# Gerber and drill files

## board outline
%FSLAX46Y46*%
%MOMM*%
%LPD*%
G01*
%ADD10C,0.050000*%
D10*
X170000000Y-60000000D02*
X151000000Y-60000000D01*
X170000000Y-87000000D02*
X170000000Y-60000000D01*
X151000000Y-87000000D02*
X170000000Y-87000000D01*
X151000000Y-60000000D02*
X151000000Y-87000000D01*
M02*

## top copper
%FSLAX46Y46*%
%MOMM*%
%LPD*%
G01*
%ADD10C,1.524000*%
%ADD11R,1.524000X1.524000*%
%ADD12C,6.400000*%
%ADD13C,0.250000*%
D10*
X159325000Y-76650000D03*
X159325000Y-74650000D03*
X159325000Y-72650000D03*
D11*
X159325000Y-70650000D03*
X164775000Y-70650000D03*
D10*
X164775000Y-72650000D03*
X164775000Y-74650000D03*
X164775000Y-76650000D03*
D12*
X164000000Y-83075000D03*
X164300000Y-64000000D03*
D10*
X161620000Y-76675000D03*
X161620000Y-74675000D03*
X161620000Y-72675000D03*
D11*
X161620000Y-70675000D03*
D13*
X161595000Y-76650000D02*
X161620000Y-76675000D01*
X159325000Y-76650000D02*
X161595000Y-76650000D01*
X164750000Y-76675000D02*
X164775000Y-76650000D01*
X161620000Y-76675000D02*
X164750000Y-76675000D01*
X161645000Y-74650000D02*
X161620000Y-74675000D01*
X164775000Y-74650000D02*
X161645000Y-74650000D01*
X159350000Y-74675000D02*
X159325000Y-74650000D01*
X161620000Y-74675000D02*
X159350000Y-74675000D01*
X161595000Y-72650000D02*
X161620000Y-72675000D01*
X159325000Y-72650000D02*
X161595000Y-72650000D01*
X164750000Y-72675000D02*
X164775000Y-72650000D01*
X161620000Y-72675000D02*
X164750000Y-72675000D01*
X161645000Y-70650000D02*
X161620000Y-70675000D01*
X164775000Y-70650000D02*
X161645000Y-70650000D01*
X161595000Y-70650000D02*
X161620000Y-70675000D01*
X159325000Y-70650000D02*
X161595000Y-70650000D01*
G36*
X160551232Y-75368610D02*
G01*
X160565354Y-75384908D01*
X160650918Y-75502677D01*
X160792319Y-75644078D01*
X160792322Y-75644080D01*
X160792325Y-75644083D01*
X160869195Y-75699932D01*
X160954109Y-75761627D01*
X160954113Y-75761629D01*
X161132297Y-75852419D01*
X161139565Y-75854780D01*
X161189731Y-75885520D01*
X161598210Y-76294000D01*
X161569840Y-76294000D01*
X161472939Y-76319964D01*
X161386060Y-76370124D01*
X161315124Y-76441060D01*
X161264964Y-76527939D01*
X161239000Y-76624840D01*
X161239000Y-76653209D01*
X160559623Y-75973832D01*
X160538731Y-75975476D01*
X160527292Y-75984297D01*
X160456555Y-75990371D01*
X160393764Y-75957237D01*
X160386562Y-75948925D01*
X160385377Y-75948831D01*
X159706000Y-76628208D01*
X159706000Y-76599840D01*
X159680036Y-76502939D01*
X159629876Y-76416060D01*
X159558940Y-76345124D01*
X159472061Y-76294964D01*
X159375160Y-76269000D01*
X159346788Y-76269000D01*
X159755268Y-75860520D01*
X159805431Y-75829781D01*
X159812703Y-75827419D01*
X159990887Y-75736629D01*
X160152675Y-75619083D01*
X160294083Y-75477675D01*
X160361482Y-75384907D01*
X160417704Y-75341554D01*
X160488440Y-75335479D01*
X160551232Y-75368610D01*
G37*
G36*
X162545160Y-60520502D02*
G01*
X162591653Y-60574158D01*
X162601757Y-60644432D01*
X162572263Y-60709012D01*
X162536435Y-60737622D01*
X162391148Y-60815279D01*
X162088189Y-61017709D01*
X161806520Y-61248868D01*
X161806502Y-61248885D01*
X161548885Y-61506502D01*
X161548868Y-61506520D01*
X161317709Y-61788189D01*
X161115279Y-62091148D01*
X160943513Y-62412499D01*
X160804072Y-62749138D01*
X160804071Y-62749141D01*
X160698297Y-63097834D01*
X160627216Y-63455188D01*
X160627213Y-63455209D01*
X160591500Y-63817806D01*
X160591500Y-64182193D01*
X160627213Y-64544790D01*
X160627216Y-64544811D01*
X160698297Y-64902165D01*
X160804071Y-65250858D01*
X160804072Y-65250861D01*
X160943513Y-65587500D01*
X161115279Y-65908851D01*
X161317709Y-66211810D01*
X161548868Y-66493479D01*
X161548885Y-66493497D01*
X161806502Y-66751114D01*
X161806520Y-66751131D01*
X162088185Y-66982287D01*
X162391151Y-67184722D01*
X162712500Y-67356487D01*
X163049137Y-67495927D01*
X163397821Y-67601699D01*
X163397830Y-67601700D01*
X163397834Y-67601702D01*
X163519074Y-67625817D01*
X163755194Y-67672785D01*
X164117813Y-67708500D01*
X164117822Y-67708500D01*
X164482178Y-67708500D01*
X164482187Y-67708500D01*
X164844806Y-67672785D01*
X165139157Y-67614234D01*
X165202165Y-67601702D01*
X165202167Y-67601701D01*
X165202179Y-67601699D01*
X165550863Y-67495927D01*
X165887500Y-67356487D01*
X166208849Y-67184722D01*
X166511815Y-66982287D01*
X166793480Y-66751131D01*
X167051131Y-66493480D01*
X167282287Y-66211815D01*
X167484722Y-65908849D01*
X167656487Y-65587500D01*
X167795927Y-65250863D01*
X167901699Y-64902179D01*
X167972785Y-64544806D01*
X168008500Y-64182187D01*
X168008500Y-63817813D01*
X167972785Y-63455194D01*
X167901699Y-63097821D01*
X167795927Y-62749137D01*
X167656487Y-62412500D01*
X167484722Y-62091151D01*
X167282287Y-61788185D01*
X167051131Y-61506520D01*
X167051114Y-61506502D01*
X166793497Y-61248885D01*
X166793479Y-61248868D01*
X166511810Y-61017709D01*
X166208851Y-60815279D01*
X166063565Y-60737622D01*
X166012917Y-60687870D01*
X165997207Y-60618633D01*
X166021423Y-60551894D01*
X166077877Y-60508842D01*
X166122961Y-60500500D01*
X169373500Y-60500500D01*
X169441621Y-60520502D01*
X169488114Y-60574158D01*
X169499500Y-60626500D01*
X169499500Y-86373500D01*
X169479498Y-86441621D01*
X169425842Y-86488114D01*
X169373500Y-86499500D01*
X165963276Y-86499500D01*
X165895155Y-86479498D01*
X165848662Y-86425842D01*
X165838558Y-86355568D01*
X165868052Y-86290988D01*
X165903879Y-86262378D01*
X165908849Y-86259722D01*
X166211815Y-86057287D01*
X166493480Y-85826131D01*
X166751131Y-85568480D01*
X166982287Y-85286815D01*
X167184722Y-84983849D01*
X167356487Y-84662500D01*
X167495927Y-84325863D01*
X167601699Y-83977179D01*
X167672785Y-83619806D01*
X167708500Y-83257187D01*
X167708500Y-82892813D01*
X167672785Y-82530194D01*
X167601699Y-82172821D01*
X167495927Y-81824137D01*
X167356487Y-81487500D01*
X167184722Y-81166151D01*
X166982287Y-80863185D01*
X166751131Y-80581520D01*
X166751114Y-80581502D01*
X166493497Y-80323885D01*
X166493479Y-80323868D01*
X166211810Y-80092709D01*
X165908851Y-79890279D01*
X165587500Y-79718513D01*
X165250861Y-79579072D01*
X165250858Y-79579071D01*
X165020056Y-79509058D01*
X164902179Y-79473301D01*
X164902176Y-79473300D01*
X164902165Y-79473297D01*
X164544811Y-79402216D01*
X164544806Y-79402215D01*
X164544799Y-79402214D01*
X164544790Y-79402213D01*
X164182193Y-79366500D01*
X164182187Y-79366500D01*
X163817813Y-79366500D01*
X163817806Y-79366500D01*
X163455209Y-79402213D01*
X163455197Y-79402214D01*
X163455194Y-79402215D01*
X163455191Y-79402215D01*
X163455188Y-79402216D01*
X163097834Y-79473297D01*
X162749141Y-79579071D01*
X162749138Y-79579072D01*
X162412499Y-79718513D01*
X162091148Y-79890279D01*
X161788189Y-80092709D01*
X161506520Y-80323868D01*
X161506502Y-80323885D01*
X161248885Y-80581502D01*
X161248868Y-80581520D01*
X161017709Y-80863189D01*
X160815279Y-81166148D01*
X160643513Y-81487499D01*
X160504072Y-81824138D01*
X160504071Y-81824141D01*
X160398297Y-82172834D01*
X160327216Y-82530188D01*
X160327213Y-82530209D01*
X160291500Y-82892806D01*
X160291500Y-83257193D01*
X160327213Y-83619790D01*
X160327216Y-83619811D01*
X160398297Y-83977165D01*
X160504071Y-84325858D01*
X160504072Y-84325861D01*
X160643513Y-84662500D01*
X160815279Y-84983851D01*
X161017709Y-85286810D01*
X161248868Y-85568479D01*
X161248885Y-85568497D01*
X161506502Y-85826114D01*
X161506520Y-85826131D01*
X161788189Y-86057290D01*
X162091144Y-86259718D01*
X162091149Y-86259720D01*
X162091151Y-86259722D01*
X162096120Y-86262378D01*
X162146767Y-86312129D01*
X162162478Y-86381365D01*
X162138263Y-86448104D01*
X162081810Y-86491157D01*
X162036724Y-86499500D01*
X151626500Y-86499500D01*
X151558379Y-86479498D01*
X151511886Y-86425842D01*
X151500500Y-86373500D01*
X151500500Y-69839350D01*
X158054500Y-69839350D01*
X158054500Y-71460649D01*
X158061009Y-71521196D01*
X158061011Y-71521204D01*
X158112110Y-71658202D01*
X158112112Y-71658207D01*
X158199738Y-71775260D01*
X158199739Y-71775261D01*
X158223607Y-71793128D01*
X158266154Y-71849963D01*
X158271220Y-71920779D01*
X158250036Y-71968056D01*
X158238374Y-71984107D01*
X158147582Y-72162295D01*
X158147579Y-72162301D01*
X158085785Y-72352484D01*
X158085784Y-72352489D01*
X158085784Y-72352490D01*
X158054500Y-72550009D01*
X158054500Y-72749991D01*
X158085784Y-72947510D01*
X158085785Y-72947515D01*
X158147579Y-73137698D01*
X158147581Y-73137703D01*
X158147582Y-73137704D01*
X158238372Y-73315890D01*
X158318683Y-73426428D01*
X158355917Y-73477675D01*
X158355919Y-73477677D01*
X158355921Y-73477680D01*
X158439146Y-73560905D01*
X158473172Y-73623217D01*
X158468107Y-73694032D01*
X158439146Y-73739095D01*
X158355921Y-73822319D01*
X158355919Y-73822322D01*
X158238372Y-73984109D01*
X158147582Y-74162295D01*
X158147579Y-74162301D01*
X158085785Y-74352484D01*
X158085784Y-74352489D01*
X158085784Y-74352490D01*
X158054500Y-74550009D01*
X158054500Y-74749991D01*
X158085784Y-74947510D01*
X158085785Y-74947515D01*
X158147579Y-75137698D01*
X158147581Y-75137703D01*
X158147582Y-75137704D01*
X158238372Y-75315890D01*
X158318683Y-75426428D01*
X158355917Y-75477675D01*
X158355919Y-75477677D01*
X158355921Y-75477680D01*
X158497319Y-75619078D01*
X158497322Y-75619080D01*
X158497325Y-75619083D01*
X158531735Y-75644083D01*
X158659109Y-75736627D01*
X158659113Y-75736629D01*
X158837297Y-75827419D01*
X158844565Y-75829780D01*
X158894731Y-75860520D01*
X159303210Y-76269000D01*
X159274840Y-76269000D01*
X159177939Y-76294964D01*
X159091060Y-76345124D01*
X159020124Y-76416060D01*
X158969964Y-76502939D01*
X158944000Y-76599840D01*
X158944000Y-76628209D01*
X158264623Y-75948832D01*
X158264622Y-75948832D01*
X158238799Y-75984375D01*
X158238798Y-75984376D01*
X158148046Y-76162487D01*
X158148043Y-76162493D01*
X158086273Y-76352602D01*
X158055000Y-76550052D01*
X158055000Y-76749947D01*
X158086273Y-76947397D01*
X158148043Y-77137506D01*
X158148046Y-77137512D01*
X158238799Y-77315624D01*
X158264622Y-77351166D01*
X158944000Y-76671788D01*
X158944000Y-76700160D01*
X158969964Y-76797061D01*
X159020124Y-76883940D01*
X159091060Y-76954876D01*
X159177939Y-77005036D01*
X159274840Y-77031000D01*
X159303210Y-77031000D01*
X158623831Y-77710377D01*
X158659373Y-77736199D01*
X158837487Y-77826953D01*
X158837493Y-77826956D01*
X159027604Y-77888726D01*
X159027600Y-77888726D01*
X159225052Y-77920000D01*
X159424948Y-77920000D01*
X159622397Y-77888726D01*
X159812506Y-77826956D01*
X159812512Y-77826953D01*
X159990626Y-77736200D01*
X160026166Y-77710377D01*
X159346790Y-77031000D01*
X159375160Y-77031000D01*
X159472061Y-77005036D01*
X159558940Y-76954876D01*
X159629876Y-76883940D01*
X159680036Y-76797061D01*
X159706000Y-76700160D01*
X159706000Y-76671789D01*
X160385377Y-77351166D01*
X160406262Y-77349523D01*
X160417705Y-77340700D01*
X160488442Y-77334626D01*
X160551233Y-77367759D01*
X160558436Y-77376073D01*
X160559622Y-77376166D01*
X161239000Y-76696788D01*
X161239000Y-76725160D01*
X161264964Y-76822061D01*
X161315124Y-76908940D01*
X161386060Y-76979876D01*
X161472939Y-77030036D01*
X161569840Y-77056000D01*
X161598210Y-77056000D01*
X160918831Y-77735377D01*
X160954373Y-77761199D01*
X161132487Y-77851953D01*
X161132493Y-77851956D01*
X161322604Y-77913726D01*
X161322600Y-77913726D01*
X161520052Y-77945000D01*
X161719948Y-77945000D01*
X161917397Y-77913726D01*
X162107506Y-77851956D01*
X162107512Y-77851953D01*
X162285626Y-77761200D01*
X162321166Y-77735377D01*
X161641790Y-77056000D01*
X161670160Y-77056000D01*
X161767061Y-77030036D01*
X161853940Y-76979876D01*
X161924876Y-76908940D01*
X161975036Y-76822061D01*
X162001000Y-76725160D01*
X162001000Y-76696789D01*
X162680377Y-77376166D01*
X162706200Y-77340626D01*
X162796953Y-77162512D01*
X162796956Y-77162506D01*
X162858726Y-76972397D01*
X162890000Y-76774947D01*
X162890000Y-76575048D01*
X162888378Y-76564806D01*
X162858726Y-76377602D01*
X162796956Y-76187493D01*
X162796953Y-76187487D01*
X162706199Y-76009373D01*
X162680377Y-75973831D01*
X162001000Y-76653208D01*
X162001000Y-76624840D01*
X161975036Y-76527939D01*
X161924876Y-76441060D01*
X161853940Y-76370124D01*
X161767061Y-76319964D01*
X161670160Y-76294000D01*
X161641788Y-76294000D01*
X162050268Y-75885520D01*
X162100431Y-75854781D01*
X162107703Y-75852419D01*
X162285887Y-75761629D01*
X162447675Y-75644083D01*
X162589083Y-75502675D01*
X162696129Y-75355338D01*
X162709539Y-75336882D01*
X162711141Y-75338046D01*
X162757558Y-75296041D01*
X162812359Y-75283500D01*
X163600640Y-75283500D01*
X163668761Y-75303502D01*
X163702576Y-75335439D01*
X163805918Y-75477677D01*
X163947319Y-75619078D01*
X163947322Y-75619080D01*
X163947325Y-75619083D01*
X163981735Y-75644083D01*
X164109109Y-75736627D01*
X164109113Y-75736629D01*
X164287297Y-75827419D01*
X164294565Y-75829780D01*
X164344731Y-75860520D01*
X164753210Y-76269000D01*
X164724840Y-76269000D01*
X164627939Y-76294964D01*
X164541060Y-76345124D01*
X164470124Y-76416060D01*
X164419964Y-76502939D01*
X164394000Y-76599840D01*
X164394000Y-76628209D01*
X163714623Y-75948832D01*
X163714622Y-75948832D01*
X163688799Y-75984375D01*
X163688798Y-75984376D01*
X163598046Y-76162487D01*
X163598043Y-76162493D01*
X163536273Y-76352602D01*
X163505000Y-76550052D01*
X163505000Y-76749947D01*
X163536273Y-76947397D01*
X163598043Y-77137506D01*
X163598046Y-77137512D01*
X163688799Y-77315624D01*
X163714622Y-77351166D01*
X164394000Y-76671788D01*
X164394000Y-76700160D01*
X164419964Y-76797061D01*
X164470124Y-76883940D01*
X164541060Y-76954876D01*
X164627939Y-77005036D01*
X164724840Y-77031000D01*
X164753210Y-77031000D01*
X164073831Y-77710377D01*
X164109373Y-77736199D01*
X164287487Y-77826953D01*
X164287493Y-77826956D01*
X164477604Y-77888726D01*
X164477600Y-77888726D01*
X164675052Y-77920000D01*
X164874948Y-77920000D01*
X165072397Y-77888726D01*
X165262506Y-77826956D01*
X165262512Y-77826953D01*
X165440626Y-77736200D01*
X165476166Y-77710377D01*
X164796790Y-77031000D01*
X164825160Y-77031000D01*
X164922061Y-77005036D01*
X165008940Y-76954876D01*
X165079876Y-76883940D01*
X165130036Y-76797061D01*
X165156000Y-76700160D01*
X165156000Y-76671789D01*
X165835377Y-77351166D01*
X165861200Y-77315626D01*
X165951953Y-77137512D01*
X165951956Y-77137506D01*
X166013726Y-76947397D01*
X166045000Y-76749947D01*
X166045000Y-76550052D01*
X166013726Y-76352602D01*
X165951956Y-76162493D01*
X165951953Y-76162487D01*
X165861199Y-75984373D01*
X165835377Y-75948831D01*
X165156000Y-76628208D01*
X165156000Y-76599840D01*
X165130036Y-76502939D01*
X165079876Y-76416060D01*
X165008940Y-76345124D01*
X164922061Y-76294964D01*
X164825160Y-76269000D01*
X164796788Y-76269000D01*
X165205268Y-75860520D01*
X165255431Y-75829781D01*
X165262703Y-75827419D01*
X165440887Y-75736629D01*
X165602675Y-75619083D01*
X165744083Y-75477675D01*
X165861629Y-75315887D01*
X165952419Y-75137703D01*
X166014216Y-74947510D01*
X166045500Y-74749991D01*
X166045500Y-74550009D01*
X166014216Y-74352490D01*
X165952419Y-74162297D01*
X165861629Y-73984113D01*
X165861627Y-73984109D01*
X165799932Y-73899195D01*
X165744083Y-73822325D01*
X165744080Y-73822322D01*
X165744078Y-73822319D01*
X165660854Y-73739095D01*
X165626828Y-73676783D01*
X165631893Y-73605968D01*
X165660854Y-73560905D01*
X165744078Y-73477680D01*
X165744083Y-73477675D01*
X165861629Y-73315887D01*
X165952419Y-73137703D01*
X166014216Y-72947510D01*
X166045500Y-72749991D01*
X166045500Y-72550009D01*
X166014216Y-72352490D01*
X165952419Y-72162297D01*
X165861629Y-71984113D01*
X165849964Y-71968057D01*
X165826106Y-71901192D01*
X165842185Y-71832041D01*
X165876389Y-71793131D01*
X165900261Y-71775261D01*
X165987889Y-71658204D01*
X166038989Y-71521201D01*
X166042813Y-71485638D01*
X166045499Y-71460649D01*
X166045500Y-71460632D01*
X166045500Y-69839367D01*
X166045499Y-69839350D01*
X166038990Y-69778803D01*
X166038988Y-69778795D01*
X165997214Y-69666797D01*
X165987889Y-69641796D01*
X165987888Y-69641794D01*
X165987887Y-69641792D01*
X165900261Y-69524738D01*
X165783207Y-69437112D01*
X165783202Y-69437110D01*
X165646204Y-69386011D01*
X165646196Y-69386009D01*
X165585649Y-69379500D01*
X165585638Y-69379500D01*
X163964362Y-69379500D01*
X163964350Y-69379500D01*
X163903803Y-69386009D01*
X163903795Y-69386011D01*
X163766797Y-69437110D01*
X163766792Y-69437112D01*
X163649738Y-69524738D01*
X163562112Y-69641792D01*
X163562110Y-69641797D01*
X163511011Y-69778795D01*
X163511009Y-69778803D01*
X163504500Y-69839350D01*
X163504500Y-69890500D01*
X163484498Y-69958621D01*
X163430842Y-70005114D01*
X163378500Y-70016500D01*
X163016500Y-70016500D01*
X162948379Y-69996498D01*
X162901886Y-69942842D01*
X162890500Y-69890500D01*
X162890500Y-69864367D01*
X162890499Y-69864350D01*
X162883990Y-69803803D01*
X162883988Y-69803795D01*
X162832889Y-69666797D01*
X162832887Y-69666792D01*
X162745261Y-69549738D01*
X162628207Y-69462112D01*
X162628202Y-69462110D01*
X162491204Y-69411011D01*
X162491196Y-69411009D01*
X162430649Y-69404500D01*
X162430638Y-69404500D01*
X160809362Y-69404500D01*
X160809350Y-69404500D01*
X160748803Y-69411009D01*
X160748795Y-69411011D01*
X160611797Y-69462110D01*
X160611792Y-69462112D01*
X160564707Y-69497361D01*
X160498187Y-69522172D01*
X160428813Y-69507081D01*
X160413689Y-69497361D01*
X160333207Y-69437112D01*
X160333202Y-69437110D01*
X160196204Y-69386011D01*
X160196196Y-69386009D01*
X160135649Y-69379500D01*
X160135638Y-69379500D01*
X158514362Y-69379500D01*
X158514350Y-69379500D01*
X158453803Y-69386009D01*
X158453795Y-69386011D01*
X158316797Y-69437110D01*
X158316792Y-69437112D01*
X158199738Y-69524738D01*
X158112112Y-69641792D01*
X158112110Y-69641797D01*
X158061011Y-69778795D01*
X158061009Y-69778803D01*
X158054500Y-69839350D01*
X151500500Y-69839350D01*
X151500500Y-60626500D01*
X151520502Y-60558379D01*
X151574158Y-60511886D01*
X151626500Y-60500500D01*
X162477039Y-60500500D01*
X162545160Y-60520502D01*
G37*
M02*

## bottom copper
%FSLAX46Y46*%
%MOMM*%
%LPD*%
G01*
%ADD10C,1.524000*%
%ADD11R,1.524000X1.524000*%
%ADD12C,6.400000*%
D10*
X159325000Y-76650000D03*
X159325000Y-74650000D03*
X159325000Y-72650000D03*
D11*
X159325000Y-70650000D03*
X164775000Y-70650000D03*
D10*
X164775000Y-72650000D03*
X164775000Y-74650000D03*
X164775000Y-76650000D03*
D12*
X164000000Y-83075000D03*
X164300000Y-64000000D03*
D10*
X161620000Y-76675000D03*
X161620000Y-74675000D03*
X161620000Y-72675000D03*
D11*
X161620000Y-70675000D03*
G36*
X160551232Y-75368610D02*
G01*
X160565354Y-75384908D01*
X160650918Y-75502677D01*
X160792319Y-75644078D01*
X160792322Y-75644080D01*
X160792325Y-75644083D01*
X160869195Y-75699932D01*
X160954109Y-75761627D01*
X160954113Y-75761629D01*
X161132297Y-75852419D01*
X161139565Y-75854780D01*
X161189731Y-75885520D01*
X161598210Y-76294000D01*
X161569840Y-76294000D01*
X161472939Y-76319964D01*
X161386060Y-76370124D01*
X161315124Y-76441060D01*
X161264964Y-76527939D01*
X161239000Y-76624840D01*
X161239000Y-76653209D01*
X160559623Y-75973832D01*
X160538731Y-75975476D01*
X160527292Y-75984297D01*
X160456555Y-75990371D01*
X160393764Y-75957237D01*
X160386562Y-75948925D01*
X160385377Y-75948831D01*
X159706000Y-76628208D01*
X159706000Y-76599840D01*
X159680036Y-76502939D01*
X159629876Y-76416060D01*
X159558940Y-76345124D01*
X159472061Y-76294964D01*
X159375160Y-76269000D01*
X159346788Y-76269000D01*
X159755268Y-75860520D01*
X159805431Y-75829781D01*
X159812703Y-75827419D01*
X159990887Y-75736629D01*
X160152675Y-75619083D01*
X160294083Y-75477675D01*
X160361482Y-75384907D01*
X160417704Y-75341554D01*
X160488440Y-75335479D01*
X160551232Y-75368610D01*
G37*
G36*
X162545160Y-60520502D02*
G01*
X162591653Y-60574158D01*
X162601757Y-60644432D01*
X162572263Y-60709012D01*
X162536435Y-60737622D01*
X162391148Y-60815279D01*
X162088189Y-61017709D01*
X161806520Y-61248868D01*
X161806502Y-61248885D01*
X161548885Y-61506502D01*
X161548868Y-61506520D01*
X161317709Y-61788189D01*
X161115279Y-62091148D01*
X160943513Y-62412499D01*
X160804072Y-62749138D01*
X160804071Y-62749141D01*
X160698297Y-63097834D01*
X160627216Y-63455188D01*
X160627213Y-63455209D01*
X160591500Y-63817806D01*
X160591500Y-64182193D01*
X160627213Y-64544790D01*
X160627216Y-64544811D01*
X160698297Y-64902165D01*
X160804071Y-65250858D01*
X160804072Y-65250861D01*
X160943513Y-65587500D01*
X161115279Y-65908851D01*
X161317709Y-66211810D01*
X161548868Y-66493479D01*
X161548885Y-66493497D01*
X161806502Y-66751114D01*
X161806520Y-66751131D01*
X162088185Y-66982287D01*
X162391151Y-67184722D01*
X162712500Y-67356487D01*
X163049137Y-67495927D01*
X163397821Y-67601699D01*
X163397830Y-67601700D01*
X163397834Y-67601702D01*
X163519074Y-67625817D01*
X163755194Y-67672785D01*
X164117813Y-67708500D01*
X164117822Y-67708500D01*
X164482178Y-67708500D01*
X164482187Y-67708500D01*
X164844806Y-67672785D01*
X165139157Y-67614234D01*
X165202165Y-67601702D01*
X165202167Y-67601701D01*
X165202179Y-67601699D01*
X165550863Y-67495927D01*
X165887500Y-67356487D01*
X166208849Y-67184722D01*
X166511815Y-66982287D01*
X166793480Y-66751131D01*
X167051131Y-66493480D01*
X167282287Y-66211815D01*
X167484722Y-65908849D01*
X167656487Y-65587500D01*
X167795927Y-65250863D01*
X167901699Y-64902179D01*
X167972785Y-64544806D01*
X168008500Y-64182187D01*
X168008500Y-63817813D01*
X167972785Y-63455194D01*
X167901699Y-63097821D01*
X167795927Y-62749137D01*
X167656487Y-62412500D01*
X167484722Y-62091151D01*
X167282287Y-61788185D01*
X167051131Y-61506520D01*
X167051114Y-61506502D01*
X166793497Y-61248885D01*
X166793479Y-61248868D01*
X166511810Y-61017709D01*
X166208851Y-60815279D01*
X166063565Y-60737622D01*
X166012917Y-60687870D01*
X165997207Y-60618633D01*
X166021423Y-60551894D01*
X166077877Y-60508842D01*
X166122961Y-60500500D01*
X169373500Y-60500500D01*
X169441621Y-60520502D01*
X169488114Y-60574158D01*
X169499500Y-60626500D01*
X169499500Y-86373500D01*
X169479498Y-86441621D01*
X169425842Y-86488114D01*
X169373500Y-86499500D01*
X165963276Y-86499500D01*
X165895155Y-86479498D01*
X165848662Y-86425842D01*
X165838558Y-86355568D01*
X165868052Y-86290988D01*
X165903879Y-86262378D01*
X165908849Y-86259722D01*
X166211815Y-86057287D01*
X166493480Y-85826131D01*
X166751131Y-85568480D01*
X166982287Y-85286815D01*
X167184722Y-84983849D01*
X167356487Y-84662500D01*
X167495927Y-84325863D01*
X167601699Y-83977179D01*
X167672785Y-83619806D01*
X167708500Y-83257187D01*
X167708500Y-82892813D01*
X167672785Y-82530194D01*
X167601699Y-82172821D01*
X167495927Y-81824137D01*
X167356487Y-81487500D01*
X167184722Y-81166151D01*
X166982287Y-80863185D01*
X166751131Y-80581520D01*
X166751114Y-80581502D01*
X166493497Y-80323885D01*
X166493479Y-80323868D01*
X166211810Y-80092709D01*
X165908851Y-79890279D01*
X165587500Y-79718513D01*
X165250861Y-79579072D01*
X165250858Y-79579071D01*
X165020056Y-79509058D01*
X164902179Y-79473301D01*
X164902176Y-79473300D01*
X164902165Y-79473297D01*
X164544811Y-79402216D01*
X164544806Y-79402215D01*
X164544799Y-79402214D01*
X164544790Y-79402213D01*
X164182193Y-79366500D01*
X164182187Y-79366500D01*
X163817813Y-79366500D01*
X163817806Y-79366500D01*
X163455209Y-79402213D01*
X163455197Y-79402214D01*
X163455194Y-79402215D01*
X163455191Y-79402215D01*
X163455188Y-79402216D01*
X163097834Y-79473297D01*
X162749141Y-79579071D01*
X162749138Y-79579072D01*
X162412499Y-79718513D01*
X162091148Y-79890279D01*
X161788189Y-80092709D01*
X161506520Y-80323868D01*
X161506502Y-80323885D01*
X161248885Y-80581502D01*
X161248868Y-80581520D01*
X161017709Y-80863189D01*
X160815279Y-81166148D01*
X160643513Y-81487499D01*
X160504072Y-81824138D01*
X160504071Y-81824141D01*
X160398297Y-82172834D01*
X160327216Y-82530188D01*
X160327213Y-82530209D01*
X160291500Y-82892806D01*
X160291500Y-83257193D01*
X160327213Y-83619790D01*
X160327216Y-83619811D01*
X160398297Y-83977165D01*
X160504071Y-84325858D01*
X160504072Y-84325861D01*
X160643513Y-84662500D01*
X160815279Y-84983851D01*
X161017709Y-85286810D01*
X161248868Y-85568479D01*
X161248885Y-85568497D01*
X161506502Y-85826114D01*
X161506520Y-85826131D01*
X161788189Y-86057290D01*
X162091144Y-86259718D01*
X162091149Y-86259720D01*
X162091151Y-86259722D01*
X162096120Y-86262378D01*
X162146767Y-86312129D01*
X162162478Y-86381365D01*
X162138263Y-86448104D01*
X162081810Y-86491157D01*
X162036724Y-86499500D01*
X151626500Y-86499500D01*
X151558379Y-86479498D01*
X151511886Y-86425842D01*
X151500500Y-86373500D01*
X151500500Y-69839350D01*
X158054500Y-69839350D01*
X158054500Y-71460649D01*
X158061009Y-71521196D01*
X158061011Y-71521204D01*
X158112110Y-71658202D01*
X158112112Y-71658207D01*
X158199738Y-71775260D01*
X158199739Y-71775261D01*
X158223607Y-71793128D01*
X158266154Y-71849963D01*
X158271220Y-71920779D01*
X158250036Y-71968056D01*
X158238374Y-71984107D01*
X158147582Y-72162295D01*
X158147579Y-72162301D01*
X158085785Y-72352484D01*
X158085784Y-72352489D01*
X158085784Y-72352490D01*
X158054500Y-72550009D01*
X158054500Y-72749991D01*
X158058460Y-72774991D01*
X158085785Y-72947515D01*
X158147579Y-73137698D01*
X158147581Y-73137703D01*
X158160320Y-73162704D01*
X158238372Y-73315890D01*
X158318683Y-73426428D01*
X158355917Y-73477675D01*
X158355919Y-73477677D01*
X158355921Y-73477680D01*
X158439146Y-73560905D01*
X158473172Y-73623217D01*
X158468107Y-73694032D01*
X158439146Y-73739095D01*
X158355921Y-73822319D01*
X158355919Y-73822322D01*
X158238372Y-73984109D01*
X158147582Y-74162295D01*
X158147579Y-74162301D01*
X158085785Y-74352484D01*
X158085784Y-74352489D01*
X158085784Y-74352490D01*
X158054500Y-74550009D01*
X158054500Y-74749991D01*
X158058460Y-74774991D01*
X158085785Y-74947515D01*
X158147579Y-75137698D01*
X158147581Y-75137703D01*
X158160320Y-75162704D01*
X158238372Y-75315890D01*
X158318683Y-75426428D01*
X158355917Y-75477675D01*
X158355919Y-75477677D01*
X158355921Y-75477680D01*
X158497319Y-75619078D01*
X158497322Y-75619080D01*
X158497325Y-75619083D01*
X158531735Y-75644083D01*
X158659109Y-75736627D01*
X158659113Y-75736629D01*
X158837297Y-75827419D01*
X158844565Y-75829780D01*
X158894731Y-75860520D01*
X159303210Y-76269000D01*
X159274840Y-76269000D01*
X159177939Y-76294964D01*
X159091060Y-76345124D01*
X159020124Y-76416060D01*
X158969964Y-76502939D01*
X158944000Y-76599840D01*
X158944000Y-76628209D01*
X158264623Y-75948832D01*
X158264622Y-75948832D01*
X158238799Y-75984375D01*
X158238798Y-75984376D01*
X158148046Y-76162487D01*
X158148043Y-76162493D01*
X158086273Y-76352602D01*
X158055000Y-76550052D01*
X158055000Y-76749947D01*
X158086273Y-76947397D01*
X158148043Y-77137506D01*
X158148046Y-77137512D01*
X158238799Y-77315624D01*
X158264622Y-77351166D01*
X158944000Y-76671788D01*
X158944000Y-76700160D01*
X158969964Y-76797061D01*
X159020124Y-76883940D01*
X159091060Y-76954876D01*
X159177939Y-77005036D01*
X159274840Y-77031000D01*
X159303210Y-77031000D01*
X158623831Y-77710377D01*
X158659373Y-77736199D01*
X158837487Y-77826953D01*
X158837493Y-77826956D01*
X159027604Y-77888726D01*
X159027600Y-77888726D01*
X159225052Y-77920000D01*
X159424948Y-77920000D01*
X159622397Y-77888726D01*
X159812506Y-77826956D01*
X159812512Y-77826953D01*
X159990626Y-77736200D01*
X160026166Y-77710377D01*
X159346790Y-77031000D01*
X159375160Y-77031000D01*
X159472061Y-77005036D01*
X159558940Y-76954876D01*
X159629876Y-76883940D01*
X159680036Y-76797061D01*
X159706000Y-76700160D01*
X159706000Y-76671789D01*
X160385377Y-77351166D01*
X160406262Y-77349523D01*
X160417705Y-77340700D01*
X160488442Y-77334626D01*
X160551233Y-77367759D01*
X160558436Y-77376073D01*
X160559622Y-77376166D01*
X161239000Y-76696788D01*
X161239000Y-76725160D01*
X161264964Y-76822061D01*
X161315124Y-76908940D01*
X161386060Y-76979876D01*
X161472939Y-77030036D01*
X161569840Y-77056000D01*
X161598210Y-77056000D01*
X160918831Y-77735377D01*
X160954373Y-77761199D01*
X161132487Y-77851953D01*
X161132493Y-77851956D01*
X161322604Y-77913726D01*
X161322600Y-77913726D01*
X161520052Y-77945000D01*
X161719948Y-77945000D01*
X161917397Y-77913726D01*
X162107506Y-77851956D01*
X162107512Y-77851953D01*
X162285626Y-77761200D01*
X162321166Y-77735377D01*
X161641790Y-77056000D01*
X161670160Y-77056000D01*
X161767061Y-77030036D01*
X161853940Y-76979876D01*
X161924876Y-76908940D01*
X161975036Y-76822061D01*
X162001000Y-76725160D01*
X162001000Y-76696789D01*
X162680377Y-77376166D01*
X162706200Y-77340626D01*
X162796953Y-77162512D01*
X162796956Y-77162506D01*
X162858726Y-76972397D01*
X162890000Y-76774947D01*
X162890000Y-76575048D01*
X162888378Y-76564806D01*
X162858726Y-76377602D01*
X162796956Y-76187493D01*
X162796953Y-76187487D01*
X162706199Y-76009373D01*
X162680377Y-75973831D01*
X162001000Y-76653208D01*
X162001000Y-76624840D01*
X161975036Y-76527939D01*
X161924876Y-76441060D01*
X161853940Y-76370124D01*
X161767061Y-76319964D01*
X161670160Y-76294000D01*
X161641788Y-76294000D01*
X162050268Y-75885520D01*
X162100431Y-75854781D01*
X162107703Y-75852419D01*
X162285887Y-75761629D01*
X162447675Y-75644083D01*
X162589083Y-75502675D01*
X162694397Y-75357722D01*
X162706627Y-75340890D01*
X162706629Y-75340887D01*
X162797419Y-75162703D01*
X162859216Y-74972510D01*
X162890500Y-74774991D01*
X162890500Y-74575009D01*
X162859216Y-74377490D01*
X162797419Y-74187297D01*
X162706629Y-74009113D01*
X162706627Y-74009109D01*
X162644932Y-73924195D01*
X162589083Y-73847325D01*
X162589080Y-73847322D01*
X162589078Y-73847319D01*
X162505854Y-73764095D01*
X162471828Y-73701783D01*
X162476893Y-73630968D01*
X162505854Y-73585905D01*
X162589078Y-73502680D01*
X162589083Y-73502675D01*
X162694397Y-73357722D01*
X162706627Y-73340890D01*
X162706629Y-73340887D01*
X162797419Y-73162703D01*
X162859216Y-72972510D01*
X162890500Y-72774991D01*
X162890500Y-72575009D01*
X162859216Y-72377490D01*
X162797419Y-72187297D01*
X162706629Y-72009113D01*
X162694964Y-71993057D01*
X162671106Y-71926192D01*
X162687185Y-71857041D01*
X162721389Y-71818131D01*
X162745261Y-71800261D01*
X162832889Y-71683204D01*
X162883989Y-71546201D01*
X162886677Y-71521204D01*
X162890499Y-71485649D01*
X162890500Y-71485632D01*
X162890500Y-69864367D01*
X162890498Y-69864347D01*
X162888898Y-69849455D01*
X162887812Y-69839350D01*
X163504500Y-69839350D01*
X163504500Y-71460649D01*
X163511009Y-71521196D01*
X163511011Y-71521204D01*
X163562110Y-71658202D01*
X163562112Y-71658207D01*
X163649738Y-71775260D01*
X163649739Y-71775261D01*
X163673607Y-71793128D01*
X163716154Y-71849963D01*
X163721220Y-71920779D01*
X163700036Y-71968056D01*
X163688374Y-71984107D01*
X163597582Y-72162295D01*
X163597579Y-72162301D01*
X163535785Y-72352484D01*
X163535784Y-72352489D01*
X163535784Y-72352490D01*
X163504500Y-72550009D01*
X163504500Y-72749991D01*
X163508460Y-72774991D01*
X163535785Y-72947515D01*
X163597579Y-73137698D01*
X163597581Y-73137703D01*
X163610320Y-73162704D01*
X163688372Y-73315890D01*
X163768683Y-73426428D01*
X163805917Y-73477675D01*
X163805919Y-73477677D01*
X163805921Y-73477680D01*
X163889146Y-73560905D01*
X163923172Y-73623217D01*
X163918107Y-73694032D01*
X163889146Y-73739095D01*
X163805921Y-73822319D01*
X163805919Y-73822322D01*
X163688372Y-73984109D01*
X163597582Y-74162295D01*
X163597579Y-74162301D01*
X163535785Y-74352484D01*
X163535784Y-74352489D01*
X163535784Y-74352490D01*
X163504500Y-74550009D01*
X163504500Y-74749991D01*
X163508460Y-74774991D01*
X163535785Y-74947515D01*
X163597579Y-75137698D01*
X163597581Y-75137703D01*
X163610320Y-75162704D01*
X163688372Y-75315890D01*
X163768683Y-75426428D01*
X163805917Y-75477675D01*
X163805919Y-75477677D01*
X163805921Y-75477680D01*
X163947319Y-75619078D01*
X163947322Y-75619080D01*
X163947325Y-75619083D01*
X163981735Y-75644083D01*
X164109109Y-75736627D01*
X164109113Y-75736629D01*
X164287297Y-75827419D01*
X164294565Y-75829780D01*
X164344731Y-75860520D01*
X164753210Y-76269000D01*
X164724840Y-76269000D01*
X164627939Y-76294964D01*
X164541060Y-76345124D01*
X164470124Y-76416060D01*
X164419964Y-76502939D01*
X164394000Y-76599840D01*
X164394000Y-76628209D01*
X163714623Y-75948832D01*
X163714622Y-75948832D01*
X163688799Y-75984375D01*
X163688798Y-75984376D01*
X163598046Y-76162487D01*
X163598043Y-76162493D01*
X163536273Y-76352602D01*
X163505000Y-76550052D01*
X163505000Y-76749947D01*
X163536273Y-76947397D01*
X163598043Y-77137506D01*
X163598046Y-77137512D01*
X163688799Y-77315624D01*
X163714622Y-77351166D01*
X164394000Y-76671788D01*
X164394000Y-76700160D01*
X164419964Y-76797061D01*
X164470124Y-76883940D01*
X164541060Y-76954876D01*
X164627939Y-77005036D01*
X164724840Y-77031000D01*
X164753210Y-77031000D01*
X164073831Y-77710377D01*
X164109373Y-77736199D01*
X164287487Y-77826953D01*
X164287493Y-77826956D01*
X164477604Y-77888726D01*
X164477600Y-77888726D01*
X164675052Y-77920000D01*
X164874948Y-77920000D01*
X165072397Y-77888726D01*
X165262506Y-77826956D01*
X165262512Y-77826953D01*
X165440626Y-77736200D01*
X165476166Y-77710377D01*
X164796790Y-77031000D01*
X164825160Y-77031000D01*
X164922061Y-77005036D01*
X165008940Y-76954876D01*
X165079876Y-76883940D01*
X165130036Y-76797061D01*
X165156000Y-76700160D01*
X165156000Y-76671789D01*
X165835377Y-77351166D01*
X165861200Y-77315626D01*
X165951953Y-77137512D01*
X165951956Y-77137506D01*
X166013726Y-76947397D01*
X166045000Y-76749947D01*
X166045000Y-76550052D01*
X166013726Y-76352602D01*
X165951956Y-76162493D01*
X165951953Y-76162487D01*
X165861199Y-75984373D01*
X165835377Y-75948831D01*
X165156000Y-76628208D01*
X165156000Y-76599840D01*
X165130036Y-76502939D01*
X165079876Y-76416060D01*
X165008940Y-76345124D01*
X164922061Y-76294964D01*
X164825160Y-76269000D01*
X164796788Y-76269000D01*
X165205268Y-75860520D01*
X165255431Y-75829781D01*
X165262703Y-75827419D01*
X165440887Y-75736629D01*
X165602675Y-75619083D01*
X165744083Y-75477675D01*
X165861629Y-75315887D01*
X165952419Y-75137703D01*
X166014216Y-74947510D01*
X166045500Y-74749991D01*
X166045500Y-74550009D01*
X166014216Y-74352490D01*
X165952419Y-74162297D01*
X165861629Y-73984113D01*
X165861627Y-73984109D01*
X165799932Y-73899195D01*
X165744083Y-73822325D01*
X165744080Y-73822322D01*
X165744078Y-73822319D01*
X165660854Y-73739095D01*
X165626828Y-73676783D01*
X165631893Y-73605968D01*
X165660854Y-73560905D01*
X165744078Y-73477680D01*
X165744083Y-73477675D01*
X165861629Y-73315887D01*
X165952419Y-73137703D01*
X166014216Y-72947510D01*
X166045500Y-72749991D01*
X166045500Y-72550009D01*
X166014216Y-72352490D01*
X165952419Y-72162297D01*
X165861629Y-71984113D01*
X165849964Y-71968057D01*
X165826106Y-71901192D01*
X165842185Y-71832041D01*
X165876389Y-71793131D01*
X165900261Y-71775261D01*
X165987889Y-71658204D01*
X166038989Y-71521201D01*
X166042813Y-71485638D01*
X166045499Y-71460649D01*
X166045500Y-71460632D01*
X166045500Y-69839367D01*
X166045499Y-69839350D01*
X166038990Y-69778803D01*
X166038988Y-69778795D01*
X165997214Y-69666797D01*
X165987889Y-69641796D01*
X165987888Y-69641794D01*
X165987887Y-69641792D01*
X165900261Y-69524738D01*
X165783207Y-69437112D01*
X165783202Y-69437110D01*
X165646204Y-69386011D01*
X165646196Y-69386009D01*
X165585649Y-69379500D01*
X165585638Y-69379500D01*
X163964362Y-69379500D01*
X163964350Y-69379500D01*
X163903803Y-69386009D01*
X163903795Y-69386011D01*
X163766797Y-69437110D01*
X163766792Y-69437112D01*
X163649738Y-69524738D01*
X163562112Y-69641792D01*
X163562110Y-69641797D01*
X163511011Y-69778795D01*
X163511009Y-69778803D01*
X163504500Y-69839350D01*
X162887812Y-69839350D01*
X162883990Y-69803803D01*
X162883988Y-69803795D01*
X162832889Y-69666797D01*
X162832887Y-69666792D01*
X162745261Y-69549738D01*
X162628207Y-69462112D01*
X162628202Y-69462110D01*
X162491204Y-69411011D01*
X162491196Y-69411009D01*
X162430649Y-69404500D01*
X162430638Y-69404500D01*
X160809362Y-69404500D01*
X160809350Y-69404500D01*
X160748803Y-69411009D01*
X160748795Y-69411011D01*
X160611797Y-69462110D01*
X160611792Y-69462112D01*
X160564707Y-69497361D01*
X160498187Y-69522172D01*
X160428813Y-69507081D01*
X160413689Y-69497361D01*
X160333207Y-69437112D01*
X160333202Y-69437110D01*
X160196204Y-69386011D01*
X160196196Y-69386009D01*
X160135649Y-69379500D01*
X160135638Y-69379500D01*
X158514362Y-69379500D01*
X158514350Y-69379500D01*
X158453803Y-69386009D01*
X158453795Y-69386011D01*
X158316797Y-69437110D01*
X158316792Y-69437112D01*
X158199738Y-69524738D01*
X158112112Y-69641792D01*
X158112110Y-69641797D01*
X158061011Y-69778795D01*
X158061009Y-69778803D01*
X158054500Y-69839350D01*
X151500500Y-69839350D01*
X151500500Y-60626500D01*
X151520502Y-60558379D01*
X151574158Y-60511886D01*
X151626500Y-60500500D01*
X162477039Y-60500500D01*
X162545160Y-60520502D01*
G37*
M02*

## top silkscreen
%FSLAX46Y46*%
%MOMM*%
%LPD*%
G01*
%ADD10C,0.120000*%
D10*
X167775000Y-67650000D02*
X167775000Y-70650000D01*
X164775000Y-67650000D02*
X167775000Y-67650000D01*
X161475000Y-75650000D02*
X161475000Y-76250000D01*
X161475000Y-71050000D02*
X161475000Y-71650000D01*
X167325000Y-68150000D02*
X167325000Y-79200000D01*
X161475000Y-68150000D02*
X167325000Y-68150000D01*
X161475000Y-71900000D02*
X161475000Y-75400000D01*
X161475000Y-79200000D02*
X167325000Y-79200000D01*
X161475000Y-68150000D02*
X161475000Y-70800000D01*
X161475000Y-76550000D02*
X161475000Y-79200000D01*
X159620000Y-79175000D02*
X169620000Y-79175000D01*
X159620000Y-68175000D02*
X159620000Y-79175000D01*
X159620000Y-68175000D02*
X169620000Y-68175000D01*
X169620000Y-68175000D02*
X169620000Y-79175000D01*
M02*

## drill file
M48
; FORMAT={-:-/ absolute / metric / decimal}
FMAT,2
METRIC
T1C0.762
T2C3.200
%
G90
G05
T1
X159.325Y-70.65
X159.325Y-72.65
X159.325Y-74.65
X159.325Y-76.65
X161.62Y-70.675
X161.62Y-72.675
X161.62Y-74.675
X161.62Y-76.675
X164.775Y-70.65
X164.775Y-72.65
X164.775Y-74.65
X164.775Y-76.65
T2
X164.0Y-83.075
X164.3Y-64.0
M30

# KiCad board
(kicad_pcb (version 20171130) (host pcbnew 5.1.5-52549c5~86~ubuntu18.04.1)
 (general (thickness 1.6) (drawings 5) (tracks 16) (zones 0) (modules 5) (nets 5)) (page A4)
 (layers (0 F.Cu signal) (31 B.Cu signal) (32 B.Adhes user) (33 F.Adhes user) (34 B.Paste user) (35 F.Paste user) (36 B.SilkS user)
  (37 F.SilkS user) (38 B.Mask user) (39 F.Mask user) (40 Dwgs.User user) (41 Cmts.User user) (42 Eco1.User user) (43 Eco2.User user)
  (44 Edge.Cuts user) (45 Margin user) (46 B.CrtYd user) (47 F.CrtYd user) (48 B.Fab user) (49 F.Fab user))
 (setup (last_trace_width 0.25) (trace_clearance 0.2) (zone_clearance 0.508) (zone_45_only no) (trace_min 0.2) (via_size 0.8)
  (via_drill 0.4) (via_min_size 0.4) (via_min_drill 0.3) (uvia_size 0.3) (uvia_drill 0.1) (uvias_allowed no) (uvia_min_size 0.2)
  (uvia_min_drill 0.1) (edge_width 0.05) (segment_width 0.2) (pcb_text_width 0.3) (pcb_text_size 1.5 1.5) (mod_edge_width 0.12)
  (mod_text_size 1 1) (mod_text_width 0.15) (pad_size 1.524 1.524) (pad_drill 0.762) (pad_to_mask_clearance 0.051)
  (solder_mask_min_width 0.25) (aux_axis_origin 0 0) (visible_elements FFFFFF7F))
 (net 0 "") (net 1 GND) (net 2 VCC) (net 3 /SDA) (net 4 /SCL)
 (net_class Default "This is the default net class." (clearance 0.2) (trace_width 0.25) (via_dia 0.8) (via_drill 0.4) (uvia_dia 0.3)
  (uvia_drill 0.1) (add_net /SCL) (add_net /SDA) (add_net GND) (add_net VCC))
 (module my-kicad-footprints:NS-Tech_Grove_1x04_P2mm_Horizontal (layer B.Cu) (at 159.325 73.65 180)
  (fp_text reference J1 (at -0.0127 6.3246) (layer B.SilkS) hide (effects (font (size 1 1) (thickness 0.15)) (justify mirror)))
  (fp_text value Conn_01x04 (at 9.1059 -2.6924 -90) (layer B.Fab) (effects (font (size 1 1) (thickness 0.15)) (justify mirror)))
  (pad 4 thru_hole circle (at 0 -3 180) (size 1.524 1.524) (drill 0.762) (layers *.Cu *.Mask) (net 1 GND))
  (pad 3 thru_hole circle (at 0 -1 180) (size 1.524 1.524) (drill 0.762) (layers *.Cu *.Mask) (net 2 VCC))
  (pad 2 thru_hole circle (at 0 1 180) (size 1.524 1.524) (drill 0.762) (layers *.Cu *.Mask) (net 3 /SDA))
  (pad 1 thru_hole rect (at 0 3 180) (size 1.524 1.524) (drill 0.762) (layers *.Cu *.Mask) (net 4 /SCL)))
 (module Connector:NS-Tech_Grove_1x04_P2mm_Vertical (layer F.Cu) (at 164.775 70.65)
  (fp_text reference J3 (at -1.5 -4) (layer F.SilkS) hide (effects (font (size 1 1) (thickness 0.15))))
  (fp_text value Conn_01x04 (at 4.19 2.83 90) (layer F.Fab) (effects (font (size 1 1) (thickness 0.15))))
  (fp_line (start 3 -3) (end 3 0) (layer F.SilkS) (width 0.12))
  (fp_line (start 0 -3) (end 3 -3) (layer F.SilkS) (width 0.12))
  (fp_line (start -3.3 5) (end -3.3 5.6) (layer F.SilkS) (width 0.12))
  (fp_line (start -3.3 0.4) (end -3.3 1) (layer F.SilkS) (width 0.12))
  (fp_line (start 2.55 -2.5) (end 2.55 8.55) (layer F.SilkS) (width 0.12))
  (fp_line (start -3.3 -2.5) (end 2.55 -2.5) (layer F.SilkS) (width 0.12))
  (fp_line (start -3.3 1.25) (end -3.3 4.75) (layer F.SilkS) (width 0.12))
  (fp_line (start -3.3 8.55) (end 2.55 8.55) (layer F.SilkS) (width 0.12))
  (fp_line (start -3.3 -2.5) (end -3.3 0.15) (layer F.SilkS) (width 0.12))
  (fp_line (start -3.3 5.9) (end -3.3 8.55) (layer F.SilkS) (width 0.12))
  (pad 1 thru_hole rect (at 0 0) (size 1.524 1.524) (drill 0.762) (layers *.Cu *.Mask) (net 4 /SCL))
  (pad 2 thru_hole circle (at 0 2) (size 1.524 1.524) (drill 0.762) (layers *.Cu *.Mask) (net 3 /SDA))
  (pad 3 thru_hole circle (at 0 4) (size 1.524 1.524) (drill 0.762) (layers *.Cu *.Mask) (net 2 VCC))
  (pad 4 thru_hole circle (at 0 6) (size 1.524 1.524) (drill 0.762) (layers *.Cu *.Mask) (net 1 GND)))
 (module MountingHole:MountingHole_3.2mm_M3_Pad (layer F.Cu) (at 164 83.075)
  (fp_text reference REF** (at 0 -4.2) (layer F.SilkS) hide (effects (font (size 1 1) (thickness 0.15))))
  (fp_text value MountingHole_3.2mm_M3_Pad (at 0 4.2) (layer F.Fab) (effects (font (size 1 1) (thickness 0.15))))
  (pad 1 thru_hole circle (at 0 0) (size 6.4 6.4) (drill 3.2) (layers *.Cu *.Mask)))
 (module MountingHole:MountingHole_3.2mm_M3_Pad (layer F.Cu) (at 164.3 64)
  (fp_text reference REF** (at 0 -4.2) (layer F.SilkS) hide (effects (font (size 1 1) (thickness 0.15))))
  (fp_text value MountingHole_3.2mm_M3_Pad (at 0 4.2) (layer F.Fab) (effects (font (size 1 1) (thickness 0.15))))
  (pad 1 thru_hole circle (at 0 0) (size 6.4 6.4) (drill 3.2) (layers *.Cu *.Mask)))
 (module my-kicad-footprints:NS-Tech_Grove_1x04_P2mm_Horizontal (layer F.Cu) (at 161.62 73.675)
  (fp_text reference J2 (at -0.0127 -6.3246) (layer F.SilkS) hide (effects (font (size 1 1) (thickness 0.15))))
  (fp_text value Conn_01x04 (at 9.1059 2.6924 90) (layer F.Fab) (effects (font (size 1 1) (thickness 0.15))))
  (fp_line (start -2 5.5) (end 8 5.5) (layer F.SilkS) (width 0.12))
  (fp_line (start -2 -5.5) (end -2 5.5) (layer F.SilkS) (width 0.12))
  (fp_line (start -2 -5.5) (end 8 -5.5) (layer F.SilkS) (width 0.12))
  (fp_line (start 8 -5.5) (end 8 5.5) (layer F.SilkS) (width 0.12))
  (pad 4 thru_hole circle (at 0 3) (size 1.524 1.524) (drill 0.762) (layers *.Cu *.Mask) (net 1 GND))
  (pad 3 thru_hole circle (at 0 1) (size 1.524 1.524) (drill 0.762) (layers *.Cu *.Mask) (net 2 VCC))
  (pad 2 thru_hole circle (at 0 -1) (size 1.524 1.524) (drill 0.762) (layers *.Cu *.Mask) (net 3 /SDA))
  (pad 1 thru_hole rect (at 0 -3) (size 1.524 1.524) (drill 0.762) (layers *.Cu *.Mask) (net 4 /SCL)))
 (gr_line (start 170 60) (end 151 60) (layer Edge.Cuts) (width 0.05))
 (gr_line (start 170 87) (end 170 60) (layer Edge.Cuts) (width 0.05))
 (gr_line (start 151 87) (end 170 87) (layer Edge.Cuts) (width 0.05))
 (gr_line (start 151 60) (end 151 87) (layer Edge.Cuts) (width 0.05))
 (segment (start 161.595 76.65) (end 161.62 76.675) (width 0.25) (layer F.Cu) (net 1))
 (segment (start 159.325 76.65) (end 161.595 76.65) (width 0.25) (layer F.Cu) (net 1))
 (segment (start 164.75 76.675) (end 164.775 76.65) (width 0.25) (layer F.Cu) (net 1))
 (segment (start 161.62 76.675) (end 164.75 76.675) (width 0.25) (layer F.Cu) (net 1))
 (segment (start 161.645 74.65) (end 161.62 74.675) (width 0.25) (layer F.Cu) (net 2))
 (segment (start 164.775 74.65) (end 161.645 74.65) (width 0.25) (layer F.Cu) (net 2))
 (segment (start 159.35 74.675) (end 159.325 74.65) (width 0.25) (layer F.Cu) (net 2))
 (segment (start 161.62 74.675) (end 159.35 74.675) (width 0.25) (layer F.Cu) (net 2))
 (segment (start 161.595 72.65) (end 161.62 72.675) (width 0.25) (layer F.Cu) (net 3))
 (segment (start 159.325 72.65) (end 161.595 72.65) (width 0.25) (layer F.Cu) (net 3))
 (segment (start 164.75 72.675) (end 164.775 72.65) (width 0.25) (layer F.Cu) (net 3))
 (segment (start 161.62 72.675) (end 164.75 72.675) (width 0.25) (layer F.Cu) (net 3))
 (segment (start 161.645 70.65) (end 161.62 70.675) (width 0.25) (layer F.Cu) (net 4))
 (segment (start 164.775 70.65) (end 161.645 70.65) (width 0.25) (layer F.Cu) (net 4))
 (segment (start 161.595 70.65) (end 161.62 70.675) (width 0.25) (layer F.Cu) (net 4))
 (segment (start 159.325 70.65) (end 161.595 70.65) (width 0.25) (layer F.Cu) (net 4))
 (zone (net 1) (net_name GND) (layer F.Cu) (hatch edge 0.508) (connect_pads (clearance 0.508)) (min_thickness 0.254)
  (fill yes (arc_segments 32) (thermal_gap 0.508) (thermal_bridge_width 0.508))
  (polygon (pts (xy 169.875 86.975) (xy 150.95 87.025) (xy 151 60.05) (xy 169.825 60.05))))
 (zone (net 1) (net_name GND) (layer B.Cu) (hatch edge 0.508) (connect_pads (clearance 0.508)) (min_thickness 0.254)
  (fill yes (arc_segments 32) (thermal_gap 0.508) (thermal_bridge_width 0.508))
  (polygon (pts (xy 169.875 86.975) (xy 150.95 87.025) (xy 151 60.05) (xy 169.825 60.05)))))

